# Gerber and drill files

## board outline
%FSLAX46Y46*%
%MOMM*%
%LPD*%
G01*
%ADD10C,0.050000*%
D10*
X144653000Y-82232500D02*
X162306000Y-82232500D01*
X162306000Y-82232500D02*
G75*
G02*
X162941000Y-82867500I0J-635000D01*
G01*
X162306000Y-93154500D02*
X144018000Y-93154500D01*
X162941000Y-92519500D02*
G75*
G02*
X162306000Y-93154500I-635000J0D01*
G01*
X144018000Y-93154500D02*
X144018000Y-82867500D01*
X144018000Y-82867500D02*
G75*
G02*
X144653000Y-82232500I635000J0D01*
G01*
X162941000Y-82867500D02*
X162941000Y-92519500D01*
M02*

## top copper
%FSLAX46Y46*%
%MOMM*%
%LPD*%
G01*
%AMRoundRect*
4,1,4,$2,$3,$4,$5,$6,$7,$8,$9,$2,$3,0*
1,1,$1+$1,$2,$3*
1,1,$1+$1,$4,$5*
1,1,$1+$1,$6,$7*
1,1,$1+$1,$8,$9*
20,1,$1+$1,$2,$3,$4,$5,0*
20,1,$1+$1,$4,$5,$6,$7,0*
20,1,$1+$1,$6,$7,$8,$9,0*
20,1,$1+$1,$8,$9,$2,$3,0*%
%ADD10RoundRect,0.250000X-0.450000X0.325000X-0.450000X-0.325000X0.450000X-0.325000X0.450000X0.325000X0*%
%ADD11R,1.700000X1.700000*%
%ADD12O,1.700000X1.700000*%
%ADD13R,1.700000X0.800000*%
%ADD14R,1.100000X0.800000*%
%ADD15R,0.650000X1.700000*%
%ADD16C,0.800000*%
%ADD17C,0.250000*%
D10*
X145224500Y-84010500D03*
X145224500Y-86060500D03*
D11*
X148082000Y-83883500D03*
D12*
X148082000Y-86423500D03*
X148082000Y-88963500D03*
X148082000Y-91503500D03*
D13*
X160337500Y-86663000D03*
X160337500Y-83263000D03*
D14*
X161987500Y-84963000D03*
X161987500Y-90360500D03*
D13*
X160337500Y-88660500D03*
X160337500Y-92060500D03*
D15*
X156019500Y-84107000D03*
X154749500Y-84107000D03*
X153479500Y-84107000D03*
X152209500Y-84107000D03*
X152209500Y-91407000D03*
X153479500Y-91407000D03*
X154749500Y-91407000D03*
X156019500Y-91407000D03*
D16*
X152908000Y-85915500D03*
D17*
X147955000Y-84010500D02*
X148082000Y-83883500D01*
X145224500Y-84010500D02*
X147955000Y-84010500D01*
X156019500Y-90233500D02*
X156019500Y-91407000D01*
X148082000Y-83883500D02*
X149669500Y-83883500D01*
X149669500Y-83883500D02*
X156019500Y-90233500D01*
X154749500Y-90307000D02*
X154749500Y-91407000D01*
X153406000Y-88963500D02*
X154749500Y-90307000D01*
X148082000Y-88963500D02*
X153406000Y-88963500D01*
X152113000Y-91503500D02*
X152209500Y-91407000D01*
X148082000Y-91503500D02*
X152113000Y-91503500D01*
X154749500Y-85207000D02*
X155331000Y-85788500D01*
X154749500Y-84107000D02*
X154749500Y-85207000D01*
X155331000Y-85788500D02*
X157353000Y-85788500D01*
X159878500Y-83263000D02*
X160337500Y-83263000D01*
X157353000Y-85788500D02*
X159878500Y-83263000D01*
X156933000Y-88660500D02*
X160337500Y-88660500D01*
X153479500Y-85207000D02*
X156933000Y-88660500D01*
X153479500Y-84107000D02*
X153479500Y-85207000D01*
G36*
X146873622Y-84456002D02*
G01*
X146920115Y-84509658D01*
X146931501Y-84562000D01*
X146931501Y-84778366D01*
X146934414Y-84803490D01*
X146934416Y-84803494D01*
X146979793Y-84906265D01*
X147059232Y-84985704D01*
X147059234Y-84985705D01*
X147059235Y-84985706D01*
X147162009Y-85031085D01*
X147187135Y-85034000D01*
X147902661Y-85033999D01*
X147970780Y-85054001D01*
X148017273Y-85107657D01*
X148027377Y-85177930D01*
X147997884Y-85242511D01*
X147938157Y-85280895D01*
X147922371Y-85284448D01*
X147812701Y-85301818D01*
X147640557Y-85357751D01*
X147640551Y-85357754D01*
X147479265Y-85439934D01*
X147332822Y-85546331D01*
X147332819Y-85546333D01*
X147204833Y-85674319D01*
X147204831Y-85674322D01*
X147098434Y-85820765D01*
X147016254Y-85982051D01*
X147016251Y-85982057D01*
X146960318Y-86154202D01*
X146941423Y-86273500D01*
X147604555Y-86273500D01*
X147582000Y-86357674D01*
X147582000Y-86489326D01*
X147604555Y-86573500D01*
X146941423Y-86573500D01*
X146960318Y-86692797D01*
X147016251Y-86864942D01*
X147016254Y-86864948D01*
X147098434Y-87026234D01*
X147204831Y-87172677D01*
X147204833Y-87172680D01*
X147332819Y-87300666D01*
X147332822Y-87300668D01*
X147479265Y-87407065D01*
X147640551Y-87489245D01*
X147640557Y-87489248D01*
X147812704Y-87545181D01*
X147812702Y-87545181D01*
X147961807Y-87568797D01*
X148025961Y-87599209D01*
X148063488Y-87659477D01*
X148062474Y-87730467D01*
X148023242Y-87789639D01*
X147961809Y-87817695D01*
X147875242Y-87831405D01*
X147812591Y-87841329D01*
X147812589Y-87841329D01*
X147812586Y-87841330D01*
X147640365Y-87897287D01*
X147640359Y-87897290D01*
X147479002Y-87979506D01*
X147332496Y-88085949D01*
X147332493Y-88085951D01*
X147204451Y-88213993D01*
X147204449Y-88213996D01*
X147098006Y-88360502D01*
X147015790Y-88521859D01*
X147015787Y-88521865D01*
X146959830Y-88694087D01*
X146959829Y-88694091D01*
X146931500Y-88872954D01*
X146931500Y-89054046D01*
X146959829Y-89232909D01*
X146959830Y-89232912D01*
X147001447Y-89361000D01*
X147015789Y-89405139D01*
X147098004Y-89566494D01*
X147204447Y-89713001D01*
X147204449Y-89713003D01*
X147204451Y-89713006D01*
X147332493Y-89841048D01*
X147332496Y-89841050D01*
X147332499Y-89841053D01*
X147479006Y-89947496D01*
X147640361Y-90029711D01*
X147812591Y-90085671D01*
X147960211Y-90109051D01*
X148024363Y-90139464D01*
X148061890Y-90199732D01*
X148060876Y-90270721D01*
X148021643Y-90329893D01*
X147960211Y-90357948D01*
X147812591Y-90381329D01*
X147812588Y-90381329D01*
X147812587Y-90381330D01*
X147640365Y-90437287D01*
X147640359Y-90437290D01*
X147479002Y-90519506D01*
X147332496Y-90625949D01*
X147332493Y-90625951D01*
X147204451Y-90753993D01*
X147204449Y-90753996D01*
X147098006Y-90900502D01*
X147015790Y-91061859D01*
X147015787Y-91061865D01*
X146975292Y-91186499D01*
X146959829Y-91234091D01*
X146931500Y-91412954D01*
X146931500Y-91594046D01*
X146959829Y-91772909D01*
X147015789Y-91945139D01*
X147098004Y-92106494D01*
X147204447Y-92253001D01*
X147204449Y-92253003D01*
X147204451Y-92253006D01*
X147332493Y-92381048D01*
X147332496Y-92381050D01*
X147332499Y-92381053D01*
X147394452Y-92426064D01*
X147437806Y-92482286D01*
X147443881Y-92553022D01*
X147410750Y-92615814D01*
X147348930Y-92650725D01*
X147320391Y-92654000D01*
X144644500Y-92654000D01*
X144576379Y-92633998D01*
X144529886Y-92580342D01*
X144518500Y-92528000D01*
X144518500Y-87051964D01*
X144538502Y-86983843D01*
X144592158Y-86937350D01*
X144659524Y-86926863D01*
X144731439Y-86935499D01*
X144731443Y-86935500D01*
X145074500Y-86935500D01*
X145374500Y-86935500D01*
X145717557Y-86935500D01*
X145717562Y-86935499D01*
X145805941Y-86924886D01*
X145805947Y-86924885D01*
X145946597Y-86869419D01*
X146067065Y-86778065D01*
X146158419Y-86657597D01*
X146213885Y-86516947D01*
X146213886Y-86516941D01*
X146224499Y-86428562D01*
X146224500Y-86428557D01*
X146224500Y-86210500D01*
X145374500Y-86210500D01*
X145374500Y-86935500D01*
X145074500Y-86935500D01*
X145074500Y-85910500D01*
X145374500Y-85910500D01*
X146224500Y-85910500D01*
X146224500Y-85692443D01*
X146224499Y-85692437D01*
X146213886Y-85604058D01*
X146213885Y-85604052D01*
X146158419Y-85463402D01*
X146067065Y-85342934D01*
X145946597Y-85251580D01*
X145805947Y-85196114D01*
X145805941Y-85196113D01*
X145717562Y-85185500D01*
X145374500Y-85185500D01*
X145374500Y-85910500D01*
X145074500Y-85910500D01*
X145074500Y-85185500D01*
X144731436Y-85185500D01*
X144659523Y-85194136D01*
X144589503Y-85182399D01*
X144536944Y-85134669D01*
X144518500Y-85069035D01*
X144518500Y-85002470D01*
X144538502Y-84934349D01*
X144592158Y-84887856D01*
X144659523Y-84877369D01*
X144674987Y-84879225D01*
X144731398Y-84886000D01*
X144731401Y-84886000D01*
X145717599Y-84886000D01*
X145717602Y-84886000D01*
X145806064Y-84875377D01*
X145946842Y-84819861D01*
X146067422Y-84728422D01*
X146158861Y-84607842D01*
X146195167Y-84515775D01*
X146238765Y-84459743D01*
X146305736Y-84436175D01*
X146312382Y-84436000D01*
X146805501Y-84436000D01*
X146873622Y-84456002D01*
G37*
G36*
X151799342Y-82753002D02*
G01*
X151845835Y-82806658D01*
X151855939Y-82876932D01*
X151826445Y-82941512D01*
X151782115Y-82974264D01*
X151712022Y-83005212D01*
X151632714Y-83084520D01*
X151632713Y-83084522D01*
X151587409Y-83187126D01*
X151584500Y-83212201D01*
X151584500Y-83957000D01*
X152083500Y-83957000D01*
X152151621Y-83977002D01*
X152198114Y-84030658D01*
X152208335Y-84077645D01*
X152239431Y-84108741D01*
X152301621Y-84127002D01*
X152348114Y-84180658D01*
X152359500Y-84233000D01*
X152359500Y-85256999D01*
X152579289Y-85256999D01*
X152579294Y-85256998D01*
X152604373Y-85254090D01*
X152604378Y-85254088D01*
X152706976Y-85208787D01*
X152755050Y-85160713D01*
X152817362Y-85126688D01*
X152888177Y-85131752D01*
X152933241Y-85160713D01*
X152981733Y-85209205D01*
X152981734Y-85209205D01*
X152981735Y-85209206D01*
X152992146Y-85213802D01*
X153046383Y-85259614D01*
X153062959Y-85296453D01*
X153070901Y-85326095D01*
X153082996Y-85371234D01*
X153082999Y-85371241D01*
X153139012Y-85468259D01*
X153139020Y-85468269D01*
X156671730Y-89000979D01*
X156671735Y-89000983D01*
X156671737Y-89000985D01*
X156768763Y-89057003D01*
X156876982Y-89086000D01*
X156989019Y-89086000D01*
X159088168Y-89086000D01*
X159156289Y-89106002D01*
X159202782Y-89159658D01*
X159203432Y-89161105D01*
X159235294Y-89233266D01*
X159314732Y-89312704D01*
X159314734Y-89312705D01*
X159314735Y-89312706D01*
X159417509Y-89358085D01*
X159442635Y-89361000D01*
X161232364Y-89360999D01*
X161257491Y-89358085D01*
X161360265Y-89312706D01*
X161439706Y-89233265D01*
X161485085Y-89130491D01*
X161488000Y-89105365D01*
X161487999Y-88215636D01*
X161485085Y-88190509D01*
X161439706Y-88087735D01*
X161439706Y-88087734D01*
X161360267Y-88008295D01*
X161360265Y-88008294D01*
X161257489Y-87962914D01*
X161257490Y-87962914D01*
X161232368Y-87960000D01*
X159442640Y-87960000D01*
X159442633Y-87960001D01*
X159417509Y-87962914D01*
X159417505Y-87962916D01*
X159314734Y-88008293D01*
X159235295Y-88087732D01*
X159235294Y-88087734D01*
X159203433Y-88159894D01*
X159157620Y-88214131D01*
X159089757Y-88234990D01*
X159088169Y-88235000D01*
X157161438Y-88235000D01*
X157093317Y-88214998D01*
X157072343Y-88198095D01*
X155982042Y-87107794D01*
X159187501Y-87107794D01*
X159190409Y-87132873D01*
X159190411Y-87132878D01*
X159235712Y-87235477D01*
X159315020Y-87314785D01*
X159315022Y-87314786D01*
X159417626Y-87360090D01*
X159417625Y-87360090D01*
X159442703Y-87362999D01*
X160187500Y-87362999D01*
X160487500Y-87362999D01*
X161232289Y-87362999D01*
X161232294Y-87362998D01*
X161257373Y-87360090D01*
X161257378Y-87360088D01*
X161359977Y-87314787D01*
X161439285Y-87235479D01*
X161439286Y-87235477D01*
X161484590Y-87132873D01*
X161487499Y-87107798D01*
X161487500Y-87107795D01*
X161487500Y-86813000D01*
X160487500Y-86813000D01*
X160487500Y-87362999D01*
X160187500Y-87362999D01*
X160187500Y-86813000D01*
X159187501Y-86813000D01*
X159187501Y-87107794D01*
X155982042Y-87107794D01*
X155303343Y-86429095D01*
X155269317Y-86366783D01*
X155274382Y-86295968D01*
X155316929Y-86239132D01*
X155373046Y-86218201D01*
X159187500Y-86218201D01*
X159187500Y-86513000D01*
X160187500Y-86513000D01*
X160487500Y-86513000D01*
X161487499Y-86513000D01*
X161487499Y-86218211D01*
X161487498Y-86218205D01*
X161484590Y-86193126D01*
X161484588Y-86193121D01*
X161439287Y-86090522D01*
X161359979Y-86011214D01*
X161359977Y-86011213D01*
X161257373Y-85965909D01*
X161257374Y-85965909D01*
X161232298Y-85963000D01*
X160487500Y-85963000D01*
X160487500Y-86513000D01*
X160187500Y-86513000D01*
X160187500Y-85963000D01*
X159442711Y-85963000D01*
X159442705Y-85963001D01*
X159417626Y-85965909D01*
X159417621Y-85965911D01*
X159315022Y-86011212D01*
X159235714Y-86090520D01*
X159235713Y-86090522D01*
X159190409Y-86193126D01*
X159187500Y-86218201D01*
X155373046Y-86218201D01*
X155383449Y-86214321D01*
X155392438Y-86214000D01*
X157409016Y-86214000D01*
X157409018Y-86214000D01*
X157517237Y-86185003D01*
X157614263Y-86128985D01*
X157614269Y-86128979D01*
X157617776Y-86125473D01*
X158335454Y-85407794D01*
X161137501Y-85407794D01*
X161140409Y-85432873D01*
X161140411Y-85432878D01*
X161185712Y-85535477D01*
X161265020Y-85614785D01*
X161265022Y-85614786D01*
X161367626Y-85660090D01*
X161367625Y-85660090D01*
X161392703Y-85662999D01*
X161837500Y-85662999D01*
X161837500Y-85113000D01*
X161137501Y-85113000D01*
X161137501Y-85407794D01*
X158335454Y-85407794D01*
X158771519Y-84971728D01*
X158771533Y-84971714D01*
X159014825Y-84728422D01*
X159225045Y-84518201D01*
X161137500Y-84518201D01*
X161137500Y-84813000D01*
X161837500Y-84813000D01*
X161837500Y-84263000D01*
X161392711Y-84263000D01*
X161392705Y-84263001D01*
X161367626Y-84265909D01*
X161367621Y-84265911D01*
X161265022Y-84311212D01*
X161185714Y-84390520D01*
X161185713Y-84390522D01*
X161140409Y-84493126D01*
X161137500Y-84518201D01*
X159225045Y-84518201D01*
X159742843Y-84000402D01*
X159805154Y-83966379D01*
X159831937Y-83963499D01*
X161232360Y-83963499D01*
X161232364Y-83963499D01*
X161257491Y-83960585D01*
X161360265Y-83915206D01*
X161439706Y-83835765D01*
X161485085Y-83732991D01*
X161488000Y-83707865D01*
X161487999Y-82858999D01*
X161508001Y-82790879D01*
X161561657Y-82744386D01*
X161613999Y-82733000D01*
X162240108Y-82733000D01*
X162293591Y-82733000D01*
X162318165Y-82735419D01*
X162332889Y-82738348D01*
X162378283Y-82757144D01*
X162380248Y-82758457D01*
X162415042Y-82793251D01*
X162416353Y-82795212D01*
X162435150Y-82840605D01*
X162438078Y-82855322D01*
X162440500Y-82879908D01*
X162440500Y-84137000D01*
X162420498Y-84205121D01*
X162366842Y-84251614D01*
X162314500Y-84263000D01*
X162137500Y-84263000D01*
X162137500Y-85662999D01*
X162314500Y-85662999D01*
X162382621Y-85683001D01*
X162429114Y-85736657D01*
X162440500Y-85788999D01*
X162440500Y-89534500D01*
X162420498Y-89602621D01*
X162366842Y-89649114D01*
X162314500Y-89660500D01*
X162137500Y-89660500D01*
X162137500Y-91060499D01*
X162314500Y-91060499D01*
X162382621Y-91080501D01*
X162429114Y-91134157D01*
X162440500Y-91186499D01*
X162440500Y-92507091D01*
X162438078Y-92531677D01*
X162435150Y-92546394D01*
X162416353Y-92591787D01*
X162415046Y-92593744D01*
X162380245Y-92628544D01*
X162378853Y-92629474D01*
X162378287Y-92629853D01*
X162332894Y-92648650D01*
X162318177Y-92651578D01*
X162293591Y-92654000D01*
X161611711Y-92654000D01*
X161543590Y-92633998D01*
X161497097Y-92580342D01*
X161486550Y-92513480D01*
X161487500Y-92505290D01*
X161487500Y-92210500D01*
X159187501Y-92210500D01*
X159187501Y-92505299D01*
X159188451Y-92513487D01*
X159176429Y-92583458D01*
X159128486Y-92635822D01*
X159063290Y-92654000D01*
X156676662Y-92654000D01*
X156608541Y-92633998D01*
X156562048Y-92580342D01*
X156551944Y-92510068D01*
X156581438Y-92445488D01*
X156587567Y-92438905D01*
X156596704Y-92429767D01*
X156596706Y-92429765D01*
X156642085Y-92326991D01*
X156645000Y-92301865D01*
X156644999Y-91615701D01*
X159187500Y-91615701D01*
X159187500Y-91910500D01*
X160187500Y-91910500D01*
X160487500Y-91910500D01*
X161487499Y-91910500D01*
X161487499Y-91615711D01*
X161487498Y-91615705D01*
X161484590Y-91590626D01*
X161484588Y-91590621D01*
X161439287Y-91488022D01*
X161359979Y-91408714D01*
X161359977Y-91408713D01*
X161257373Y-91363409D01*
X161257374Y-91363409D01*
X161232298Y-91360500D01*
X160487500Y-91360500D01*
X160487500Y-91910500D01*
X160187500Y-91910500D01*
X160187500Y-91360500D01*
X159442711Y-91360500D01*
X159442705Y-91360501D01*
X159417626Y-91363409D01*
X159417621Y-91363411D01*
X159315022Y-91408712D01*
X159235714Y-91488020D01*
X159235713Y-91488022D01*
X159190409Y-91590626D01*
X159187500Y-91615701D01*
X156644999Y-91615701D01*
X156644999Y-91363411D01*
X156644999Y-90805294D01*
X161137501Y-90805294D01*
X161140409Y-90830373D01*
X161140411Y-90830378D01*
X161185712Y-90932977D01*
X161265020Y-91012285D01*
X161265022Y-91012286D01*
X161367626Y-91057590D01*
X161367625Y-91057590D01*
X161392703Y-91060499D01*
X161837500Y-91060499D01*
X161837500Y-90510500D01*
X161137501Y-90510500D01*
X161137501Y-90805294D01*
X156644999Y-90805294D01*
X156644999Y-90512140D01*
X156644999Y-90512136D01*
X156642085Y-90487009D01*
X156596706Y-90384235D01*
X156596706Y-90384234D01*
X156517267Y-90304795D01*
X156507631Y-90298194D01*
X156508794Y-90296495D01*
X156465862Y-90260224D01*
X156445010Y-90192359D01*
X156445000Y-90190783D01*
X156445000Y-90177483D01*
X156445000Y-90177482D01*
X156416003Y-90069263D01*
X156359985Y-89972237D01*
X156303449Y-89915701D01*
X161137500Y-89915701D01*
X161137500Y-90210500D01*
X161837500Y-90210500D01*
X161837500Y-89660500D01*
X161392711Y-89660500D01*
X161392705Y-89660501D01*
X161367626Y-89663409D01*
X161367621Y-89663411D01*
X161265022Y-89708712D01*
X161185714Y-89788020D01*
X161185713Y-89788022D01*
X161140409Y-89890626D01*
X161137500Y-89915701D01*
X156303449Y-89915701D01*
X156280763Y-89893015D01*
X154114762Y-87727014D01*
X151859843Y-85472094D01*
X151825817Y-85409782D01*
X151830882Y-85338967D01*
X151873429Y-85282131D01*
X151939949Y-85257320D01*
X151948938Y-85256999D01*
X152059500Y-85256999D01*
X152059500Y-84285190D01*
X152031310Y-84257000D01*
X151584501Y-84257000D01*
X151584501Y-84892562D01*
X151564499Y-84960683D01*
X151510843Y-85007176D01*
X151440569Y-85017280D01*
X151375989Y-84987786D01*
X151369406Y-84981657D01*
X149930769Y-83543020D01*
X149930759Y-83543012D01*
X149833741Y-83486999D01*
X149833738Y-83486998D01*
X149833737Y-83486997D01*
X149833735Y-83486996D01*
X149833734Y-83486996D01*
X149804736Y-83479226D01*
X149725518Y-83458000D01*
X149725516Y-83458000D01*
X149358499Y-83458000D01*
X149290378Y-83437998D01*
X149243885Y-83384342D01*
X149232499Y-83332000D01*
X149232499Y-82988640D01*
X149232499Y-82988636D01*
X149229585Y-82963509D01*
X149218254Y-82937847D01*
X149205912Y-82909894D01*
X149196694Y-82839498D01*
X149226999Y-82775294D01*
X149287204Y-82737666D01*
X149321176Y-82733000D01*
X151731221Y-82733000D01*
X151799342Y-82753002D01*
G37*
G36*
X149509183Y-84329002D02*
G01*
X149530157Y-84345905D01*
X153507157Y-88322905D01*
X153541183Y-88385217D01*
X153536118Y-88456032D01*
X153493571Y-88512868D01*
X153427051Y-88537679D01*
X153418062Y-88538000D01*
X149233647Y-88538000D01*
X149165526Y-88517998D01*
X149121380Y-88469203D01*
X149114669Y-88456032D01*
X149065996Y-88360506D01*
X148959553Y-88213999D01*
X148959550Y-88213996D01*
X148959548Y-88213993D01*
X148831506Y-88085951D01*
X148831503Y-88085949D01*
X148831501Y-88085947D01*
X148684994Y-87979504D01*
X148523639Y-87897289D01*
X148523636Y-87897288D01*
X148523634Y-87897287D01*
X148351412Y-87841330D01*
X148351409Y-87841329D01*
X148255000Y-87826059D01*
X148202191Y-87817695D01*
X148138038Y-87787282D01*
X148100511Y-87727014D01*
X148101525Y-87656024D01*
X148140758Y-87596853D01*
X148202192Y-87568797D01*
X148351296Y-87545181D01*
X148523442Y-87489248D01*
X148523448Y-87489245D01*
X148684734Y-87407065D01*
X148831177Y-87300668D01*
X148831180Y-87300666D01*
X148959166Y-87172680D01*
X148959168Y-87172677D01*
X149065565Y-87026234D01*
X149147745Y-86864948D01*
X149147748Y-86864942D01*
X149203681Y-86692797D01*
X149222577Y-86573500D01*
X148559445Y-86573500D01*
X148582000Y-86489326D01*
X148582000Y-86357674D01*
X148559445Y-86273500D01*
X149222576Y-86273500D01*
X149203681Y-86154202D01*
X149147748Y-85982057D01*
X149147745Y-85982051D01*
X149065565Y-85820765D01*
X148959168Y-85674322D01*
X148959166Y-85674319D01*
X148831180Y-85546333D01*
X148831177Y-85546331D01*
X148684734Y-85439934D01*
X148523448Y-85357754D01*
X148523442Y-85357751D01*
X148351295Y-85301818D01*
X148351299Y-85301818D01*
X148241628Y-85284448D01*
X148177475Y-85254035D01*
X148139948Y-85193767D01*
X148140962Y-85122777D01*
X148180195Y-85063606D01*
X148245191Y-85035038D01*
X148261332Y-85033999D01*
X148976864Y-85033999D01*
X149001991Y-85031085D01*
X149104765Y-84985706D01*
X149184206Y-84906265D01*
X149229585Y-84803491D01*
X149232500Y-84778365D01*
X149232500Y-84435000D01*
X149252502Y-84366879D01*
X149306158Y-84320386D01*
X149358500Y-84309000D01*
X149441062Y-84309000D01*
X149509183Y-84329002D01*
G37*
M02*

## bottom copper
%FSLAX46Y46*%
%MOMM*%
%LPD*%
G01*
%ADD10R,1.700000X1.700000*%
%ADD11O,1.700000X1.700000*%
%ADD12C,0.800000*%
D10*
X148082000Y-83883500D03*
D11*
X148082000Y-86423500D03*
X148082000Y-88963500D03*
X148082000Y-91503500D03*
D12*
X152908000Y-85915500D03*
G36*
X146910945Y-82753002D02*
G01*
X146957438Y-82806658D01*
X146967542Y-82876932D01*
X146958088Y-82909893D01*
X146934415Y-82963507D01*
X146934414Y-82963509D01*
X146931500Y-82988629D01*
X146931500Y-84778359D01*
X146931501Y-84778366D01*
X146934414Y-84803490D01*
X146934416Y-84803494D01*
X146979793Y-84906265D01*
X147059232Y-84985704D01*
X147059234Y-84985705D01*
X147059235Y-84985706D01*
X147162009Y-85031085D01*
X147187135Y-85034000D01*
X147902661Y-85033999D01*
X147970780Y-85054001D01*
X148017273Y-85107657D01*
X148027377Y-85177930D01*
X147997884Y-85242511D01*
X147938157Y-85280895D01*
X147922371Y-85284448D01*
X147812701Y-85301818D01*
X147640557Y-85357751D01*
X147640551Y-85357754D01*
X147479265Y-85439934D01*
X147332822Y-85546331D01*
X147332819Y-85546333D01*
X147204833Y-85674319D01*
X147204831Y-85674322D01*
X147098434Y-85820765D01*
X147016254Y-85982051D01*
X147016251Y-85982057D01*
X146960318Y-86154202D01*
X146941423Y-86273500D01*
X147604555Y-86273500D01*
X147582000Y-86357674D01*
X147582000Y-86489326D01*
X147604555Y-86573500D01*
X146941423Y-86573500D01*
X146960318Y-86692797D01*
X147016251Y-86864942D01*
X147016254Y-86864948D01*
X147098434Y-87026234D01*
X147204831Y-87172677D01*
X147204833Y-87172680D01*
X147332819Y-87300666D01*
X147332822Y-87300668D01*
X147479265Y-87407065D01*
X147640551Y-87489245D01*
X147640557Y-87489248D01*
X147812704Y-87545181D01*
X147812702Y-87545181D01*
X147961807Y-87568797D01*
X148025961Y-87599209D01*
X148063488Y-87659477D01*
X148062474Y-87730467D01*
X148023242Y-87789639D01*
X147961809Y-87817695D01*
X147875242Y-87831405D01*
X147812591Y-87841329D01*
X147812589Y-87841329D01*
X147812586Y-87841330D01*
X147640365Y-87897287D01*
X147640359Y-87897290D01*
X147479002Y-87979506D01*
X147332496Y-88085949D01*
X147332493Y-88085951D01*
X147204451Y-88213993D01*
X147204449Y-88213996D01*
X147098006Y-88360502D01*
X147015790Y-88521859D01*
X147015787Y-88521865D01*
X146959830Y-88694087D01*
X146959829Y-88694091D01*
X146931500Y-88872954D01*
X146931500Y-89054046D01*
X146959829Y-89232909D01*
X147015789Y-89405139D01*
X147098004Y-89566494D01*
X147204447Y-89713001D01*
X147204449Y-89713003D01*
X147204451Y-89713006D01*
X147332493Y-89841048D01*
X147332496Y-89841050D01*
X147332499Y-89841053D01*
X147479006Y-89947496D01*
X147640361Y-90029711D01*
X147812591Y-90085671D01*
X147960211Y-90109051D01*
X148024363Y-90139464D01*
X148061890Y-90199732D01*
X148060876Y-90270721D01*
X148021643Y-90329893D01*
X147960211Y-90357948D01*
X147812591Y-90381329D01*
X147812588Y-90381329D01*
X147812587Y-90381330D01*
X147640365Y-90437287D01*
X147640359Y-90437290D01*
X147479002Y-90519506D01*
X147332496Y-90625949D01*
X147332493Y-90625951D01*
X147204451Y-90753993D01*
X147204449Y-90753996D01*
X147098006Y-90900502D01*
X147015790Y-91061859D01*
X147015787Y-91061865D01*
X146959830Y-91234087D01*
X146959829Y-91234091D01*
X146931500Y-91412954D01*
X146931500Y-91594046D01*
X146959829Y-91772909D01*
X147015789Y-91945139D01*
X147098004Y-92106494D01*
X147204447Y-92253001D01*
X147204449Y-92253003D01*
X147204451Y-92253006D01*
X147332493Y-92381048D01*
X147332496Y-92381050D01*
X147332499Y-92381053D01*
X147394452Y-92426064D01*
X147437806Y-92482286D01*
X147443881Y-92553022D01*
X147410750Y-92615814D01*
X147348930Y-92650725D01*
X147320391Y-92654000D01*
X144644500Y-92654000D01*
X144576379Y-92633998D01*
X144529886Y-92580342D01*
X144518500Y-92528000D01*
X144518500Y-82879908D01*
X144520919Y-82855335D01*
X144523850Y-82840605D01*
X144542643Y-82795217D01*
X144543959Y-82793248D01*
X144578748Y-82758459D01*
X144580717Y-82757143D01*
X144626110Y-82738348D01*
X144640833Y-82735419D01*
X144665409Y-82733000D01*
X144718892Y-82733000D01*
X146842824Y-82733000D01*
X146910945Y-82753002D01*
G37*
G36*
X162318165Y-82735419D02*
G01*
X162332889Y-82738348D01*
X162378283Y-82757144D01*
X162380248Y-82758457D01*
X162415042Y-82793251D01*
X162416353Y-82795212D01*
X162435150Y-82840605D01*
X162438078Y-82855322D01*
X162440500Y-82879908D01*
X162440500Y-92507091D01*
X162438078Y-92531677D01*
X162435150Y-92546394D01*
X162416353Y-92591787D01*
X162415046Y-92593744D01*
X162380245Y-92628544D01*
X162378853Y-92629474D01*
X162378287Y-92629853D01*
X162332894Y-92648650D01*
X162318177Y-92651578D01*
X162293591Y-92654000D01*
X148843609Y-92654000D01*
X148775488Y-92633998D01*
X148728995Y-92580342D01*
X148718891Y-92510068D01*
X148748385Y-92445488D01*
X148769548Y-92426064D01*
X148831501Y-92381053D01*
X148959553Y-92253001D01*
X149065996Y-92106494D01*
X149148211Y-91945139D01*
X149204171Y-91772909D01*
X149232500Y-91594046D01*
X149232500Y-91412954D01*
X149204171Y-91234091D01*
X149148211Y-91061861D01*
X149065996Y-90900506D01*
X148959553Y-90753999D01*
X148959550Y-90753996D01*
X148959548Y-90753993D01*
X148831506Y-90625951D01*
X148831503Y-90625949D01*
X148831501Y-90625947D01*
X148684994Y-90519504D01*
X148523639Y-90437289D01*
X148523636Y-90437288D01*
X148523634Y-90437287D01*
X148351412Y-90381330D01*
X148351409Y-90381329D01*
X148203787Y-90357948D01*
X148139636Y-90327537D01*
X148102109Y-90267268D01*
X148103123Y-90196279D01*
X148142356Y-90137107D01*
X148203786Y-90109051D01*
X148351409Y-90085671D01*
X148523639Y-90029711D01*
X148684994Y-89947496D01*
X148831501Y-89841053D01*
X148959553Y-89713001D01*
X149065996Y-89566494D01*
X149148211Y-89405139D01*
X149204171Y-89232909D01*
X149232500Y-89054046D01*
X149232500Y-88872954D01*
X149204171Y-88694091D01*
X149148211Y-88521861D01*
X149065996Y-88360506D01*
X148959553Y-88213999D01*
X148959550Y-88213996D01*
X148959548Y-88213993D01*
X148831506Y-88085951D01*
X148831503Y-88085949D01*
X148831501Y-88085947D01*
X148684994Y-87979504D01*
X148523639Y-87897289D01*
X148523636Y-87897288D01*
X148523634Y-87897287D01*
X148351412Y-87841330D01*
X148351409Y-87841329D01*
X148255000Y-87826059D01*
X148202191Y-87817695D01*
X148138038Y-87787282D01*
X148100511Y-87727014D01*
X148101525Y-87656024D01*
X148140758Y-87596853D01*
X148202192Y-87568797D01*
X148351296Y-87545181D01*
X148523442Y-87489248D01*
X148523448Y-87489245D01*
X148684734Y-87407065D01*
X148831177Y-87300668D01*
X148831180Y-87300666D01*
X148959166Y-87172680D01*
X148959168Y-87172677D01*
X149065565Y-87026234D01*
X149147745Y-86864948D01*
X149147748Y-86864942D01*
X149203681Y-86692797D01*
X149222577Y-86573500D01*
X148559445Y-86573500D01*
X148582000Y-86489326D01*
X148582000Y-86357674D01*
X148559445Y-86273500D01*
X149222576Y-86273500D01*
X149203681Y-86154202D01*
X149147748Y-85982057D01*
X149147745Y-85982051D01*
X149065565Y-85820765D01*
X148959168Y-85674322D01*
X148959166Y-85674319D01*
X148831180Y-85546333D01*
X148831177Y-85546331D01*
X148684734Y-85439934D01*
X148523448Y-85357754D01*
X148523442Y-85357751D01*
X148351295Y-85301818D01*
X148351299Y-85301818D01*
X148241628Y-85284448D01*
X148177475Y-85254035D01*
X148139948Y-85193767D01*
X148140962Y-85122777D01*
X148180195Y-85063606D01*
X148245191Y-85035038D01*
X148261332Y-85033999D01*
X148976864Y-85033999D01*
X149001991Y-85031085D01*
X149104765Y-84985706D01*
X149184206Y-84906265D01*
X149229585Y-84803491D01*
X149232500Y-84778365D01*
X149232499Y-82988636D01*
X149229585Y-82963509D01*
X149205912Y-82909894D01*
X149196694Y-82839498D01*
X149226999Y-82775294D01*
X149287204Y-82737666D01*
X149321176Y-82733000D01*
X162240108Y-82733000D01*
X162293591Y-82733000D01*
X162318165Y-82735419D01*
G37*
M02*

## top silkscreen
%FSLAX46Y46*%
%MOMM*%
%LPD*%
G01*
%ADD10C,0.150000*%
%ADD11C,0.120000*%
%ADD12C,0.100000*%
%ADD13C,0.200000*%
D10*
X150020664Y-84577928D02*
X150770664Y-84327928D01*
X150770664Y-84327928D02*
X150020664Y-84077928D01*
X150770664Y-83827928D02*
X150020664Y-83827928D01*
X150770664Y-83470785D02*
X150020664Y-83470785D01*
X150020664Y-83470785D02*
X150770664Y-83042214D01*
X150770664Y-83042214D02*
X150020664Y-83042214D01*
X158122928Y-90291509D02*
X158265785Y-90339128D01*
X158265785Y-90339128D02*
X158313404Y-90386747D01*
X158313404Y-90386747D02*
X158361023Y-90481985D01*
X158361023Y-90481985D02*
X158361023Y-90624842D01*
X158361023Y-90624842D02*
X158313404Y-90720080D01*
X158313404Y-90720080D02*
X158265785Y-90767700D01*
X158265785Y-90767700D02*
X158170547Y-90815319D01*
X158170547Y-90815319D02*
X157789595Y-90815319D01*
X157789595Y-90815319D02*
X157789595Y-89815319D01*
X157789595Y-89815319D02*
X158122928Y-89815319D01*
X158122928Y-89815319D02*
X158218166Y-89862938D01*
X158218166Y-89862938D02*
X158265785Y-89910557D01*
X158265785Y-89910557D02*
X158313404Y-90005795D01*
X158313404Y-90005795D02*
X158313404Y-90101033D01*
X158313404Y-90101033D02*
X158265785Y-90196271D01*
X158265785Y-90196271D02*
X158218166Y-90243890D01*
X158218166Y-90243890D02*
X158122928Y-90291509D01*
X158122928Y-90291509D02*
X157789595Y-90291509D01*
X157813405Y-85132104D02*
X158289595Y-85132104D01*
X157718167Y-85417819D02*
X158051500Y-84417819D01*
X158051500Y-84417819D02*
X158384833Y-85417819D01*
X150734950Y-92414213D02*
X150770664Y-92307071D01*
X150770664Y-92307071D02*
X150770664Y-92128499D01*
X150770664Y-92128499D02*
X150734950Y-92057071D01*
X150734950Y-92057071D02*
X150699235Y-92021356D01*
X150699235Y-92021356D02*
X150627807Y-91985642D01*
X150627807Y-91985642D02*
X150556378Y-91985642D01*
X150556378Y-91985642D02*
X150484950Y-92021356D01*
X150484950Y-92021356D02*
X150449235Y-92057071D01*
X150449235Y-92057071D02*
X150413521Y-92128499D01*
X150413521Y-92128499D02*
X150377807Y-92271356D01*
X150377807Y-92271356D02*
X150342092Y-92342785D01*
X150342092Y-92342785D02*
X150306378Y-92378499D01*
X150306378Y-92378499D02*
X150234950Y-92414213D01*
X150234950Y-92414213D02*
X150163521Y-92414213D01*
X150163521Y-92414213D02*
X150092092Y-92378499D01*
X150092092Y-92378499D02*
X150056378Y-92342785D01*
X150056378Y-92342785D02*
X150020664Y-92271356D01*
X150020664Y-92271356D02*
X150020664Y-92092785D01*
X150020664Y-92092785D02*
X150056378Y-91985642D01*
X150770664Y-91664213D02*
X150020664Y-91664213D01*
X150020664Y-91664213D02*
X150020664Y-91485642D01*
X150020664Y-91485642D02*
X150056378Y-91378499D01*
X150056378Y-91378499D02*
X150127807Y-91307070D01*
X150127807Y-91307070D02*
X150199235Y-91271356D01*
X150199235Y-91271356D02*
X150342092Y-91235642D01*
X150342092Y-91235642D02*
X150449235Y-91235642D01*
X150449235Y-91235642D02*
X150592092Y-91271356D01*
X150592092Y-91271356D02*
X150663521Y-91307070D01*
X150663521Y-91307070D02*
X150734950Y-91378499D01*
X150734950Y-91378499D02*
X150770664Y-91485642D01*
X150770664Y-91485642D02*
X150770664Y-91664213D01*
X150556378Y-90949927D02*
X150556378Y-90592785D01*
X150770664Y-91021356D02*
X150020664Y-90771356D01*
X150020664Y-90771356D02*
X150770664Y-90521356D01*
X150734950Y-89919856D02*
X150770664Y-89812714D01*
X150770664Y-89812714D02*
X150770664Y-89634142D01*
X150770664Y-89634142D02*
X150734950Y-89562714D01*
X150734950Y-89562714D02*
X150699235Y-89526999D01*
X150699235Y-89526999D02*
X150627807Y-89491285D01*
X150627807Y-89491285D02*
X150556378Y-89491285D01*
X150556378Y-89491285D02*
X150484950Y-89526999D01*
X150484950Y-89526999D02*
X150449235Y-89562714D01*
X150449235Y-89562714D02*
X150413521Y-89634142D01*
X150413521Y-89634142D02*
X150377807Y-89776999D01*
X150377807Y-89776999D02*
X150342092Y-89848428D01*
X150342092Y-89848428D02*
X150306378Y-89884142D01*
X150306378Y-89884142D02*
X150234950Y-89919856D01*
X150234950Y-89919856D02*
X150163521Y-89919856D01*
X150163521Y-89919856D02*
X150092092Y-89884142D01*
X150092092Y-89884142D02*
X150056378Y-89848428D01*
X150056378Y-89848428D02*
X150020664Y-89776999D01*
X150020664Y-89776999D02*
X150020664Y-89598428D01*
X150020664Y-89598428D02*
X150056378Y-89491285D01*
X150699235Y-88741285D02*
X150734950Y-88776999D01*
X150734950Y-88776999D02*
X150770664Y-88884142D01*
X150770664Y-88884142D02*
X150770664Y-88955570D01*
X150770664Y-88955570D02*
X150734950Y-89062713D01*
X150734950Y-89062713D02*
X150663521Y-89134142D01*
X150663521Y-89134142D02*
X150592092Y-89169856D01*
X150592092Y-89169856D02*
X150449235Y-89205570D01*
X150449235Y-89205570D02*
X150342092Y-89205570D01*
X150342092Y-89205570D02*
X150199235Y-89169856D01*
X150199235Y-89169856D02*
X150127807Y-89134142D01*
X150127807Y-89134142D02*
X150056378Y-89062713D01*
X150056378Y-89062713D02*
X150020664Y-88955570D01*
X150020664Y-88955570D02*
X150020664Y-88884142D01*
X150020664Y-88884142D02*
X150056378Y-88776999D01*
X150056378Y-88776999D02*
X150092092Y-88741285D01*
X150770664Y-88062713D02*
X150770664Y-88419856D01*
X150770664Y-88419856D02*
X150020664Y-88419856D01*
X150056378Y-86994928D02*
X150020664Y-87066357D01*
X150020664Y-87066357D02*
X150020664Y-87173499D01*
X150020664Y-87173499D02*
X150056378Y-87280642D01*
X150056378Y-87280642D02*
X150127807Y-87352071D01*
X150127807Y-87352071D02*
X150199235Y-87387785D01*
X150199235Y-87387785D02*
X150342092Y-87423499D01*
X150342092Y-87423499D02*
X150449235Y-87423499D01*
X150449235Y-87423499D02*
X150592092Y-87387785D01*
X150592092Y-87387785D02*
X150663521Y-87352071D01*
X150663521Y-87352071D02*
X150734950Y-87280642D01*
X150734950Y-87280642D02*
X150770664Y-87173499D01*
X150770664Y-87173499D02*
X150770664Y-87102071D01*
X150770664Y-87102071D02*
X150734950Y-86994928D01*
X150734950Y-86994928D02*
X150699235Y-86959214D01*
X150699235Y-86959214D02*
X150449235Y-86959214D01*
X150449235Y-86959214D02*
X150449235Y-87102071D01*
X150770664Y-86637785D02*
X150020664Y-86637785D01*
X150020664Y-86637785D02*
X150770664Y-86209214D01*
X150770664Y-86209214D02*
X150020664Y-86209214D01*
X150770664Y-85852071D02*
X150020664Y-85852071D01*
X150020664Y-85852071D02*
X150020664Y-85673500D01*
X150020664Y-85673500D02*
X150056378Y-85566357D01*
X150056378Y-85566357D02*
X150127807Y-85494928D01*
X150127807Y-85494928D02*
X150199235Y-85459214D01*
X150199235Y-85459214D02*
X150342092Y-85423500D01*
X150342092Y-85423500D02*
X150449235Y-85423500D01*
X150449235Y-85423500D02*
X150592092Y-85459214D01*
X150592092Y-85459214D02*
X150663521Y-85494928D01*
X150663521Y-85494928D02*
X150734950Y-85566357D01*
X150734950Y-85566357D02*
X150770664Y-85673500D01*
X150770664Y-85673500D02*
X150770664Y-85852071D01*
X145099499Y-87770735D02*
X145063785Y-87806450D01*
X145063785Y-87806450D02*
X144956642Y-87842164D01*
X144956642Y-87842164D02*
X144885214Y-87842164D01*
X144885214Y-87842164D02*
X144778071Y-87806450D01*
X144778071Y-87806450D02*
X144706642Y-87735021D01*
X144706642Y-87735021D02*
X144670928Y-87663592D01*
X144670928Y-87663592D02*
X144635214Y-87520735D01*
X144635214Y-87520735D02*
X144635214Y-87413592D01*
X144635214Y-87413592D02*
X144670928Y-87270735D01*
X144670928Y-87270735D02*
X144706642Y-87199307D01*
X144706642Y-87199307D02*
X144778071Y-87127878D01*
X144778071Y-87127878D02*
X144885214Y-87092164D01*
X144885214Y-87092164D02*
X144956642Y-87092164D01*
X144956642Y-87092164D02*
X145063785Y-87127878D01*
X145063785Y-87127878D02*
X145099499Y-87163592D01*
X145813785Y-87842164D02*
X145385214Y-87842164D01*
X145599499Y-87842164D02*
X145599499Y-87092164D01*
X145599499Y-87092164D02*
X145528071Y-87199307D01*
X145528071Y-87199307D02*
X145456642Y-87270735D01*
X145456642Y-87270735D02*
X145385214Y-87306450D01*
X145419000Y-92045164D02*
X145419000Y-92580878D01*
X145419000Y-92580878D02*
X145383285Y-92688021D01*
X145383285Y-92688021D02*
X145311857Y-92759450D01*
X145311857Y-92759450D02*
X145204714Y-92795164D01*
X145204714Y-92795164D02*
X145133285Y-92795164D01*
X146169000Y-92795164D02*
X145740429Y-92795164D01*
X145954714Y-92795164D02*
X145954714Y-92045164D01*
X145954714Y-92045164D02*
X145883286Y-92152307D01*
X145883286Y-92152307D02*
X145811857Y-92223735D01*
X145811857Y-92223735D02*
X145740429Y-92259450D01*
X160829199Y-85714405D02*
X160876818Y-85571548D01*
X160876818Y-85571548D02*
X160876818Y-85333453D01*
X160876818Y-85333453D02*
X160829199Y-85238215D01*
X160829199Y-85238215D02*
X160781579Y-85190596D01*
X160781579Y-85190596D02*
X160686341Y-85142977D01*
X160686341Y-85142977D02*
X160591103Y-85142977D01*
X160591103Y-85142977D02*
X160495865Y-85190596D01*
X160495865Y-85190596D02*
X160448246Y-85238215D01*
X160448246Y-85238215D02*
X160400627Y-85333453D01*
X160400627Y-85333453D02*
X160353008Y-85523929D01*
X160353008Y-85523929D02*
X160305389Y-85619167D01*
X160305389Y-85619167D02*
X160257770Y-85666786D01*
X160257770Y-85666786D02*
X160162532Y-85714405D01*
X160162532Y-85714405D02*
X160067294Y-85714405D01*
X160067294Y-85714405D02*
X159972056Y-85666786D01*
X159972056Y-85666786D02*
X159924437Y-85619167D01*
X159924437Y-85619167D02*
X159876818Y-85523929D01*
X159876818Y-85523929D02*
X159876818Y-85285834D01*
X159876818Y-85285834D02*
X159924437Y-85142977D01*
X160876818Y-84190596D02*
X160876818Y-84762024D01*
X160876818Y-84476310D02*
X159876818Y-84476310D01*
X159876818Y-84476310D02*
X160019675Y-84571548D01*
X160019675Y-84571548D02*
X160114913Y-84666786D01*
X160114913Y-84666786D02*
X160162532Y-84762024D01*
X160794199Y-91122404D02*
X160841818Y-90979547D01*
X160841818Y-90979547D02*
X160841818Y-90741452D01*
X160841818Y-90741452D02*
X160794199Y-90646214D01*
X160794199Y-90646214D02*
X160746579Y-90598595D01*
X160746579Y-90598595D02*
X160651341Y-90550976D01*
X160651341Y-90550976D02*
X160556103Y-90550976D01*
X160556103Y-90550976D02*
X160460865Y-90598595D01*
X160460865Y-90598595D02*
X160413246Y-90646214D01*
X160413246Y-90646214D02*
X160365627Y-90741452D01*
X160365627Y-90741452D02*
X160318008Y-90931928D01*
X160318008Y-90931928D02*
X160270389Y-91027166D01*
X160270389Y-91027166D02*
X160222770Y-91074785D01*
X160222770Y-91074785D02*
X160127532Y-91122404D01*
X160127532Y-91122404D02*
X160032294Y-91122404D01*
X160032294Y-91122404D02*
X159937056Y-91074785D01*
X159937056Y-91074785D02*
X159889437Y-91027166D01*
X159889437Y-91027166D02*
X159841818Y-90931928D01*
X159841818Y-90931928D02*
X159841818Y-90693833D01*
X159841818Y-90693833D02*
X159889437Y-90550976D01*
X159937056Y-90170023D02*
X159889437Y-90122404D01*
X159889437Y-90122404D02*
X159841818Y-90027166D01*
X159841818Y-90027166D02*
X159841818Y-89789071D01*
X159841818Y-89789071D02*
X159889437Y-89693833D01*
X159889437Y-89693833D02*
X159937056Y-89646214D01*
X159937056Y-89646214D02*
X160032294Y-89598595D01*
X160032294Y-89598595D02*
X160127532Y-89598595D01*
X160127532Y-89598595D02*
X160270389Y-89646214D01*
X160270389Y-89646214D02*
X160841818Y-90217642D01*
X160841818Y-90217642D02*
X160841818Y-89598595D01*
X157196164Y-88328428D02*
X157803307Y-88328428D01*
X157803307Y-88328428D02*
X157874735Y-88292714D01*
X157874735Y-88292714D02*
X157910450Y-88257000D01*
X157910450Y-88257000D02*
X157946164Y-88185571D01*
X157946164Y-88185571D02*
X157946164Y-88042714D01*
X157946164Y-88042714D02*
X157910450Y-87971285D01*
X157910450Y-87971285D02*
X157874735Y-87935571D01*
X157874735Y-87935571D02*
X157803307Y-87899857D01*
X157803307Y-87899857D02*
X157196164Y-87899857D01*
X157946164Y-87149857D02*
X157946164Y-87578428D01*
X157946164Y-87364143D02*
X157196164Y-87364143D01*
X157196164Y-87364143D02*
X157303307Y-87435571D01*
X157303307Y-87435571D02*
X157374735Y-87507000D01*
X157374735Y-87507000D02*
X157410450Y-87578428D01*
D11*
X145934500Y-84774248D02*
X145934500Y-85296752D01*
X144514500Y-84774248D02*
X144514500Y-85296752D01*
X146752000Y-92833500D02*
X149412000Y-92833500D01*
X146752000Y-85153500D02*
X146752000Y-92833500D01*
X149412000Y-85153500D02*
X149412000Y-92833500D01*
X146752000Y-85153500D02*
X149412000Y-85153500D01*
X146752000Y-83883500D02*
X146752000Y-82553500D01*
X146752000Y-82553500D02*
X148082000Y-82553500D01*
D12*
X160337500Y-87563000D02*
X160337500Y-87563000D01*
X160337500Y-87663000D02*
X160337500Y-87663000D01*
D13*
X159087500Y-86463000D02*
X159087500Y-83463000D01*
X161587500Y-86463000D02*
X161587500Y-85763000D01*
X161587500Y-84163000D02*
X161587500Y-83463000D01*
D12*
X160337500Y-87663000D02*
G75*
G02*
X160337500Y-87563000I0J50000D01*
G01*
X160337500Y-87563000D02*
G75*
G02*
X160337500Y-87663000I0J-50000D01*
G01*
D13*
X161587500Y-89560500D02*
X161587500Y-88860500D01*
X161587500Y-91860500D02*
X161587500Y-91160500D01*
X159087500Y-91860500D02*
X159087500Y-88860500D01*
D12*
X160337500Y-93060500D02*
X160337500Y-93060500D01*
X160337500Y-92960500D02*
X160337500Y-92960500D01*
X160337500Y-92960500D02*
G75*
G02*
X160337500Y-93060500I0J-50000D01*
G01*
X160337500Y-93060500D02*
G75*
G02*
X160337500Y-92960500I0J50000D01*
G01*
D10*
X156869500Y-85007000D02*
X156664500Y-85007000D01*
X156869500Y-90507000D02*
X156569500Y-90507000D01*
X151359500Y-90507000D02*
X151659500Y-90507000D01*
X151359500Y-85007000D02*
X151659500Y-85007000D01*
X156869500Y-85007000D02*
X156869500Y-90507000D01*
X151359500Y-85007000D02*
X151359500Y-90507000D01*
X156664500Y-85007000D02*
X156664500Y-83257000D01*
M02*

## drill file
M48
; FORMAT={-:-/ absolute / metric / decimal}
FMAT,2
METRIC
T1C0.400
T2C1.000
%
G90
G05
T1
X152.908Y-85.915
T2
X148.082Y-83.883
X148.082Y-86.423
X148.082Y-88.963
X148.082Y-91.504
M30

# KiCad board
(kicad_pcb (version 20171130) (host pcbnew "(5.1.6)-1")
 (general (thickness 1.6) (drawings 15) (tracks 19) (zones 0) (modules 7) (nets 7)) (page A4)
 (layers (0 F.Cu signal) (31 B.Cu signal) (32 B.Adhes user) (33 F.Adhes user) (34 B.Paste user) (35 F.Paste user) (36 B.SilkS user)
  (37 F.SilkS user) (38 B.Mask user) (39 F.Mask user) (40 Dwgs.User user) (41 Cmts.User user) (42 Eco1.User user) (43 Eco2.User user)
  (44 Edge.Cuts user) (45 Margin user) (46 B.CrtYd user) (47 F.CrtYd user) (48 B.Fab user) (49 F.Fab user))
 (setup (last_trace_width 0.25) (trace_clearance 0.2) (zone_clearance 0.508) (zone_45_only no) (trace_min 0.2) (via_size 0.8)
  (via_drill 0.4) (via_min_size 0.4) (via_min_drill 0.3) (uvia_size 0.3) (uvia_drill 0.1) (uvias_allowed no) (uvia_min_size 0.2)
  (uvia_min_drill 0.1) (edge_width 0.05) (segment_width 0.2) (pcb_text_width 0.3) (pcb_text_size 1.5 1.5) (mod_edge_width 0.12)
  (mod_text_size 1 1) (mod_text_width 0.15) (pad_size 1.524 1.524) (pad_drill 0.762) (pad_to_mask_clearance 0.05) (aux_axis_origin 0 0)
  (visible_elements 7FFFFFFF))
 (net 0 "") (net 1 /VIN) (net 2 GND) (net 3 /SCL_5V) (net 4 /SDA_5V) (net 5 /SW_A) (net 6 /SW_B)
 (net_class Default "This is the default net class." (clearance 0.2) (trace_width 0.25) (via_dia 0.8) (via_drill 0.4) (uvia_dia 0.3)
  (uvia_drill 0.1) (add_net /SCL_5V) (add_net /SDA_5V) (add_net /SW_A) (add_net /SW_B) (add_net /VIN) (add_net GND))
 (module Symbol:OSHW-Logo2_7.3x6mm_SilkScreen (layer B.Cu) (at 159.512 88.519 180)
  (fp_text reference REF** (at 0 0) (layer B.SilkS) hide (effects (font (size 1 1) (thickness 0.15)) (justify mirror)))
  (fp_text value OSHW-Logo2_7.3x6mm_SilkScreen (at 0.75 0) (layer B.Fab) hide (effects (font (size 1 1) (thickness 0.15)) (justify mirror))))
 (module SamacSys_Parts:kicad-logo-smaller (layer B.Cu) (at 153.0985 88.265 180)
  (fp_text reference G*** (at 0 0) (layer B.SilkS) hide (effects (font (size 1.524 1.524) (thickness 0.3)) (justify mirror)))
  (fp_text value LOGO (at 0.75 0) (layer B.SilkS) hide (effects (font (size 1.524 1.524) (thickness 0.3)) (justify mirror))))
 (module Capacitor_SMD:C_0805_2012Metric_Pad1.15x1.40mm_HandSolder (layer F.Cu) (at 145.2245 85.0355 270)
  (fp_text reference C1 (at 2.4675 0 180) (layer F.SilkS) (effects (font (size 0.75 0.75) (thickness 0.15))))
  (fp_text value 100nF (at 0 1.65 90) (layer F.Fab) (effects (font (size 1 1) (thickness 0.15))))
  (fp_line (start -0.261252 -0.71) (end 0.261252 -0.71) (layer F.SilkS) (width 0.12))
  (fp_line (start -0.261252 0.71) (end 0.261252 0.71) (layer F.SilkS) (width 0.12))
  (pad 1 smd roundrect (at -1.025 0 270) (size 1.15 1.4) (layers F.Cu F.Paste F.Mask) (roundrect_rratio 0.217391) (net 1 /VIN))
  (pad 2 smd roundrect (at 1.025 0 270) (size 1.15 1.4) (layers F.Cu F.Paste F.Mask) (roundrect_rratio 0.217391) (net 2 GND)))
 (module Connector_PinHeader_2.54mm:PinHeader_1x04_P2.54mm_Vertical (layer F.Cu) (at 148.082 83.8835)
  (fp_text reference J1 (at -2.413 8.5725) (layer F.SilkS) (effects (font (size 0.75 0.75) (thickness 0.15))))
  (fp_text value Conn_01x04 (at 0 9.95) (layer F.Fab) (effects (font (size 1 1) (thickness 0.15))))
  (fp_line (start -1.33 8.95) (end 1.33 8.95) (layer F.SilkS) (width 0.12))
  (fp_line (start -1.33 1.27) (end -1.33 8.95) (layer F.SilkS) (width 0.12))
  (fp_line (start 1.33 1.27) (end 1.33 8.95) (layer F.SilkS) (width 0.12))
  (fp_line (start -1.33 1.27) (end 1.33 1.27) (layer F.SilkS) (width 0.12))
  (fp_line (start -1.33 0) (end -1.33 -1.33) (layer F.SilkS) (width 0.12))
  (fp_line (start -1.33 -1.33) (end 0 -1.33) (layer F.SilkS) (width 0.12))
  (pad 1 thru_hole rect (at 0 0) (size 1.7 1.7) (drill 1) (layers *.Cu *.Mask) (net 1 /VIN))
  (pad 2 thru_hole oval (at 0 2.54) (size 1.7 1.7) (drill 1) (layers *.Cu *.Mask) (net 2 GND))
  (pad 3 thru_hole oval (at 0 5.08) (size 1.7 1.7) (drill 1) (layers *.Cu *.Mask) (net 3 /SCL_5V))
  (pad 4 thru_hole oval (at 0 7.62) (size 1.7 1.7) (drill 1) (layers *.Cu *.Mask) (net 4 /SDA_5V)))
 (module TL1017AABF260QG (layer F.Cu) (at 160.3375 84.963 90)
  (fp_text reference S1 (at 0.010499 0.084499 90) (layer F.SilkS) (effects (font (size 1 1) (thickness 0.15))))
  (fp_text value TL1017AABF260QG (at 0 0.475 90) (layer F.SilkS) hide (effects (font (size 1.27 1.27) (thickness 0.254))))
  (fp_line (start -2.6 0) (end -2.6 0) (layer F.SilkS) (width 0.1))
  (fp_line (start -2.7 0) (end -2.7 0) (layer F.SilkS) (width 0.1))
  (fp_line (start -1.5 -1.25) (end 1.5 -1.25) (layer F.SilkS) (width 0.2))
  (fp_line (start -1.5 1.25) (end -0.8 1.25) (layer F.SilkS) (width 0.2))
  (fp_line (start 0.8 1.25) (end 1.5 1.25) (layer F.SilkS) (width 0.2))
  (fp_arc (start -2.65 0) (end -2.6 0) (angle -180) (layer F.SilkS) (width 0.1))
  (fp_arc (start -2.65 0) (end -2.7 0) (angle -180) (layer F.SilkS) (width 0.1))
  (pad 1 smd rect (at -1.7 0 90) (size 0.8 1.7) (layers F.Cu F.Paste F.Mask) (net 2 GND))
  (pad 2 smd rect (at 1.7 0 90) (size 0.8 1.7) (layers F.Cu F.Paste F.Mask) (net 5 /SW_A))
  (pad G1 smd rect (at 0 1.65 90) (size 0.8 1.1) (layers F.Cu F.Paste F.Mask) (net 2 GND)))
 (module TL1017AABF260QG (layer F.Cu) (at 160.3375 90.3605 90)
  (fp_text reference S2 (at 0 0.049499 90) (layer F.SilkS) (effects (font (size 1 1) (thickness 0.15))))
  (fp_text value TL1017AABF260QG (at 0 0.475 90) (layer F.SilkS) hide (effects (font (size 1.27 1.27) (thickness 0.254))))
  (fp_line (start 0.8 1.25) (end 1.5 1.25) (layer F.SilkS) (width 0.2))
  (fp_line (start -1.5 1.25) (end -0.8 1.25) (layer F.SilkS) (width 0.2))
  (fp_line (start -1.5 -1.25) (end 1.5 -1.25) (layer F.SilkS) (width 0.2))
  (fp_line (start -2.7 0) (end -2.7 0) (layer F.SilkS) (width 0.1))
  (fp_line (start -2.6 0) (end -2.6 0) (layer F.SilkS) (width 0.1))
  (fp_arc (start -2.65 0) (end -2.7 0) (angle -180) (layer F.SilkS) (width 0.1))
  (fp_arc (start -2.65 0) (end -2.6 0) (angle -180) (layer F.SilkS) (width 0.1))
  (pad G1 smd rect (at 0 1.65 90) (size 0.8 1.1) (layers F.Cu F.Paste F.Mask) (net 2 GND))
  (pad 2 smd rect (at 1.7 0 90) (size 0.8 1.7) (layers F.Cu F.Paste F.Mask) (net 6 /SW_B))
  (pad 1 smd rect (at -1.7 0 90) (size 0.8 1.7) (layers F.Cu F.Paste F.Mask) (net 2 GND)))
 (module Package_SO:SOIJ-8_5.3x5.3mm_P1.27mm (layer F.Cu) (at 154.1145 87.757 270)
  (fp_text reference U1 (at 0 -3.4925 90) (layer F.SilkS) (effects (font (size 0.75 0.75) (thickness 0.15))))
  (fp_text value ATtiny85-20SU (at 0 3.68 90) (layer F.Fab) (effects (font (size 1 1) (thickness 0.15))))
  (fp_line (start -2.75 -2.755) (end -2.75 -2.55) (layer F.SilkS) (width 0.15))
  (fp_line (start 2.75 -2.755) (end 2.75 -2.455) (layer F.SilkS) (width 0.15))
  (fp_line (start 2.75 2.755) (end 2.75 2.455) (layer F.SilkS) (width 0.15))
  (fp_line (start -2.75 2.755) (end -2.75 2.455) (layer F.SilkS) (width 0.15))
  (fp_line (start -2.75 -2.755) (end 2.75 -2.755) (layer F.SilkS) (width 0.15))
  (fp_line (start -2.75 2.755) (end 2.75 2.755) (layer F.SilkS) (width 0.15))
  (fp_line (start -2.75 -2.55) (end -4.5 -2.55) (layer F.SilkS) (width 0.15))
  (pad 1 smd rect (at -3.65 -1.905 270) (size 1.7 0.65) (layers F.Cu F.Paste F.Mask))
  (pad 2 smd rect (at -3.65 -0.635 270) (size 1.7 0.65) (layers F.Cu F.Paste F.Mask) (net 5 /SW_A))
  (pad 3 smd rect (at -3.65 0.635 270) (size 1.7 0.65) (layers F.Cu F.Paste F.Mask) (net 6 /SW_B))
  (pad 4 smd rect (at -3.65 1.905 270) (size 1.7 0.65) (layers F.Cu F.Paste F.Mask) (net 2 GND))
  (pad 5 smd rect (at 3.65 1.905 270) (size 1.7 0.65) (layers F.Cu F.Paste F.Mask) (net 4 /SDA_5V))
  (pad 6 smd rect (at 3.65 0.635 270) (size 1.7 0.65) (layers F.Cu F.Paste F.Mask))
  (pad 7 smd rect (at 3.65 -0.635 270) (size 1.7 0.65) (layers F.Cu F.Paste F.Mask) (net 3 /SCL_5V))
  (pad 8 smd rect (at 3.65 -1.905 270) (size 1.7 0.65) (layers F.Cu F.Paste F.Mask) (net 1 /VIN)))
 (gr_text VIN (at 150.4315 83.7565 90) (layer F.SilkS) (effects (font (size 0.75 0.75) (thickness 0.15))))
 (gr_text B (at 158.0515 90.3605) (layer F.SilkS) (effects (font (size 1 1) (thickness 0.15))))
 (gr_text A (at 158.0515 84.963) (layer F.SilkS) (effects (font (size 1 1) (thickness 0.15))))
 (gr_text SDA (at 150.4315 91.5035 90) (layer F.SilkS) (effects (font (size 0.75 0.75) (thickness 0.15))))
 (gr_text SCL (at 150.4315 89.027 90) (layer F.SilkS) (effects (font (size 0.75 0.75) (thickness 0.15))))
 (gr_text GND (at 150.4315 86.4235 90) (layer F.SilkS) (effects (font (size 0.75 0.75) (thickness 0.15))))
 (gr_line (start 144.653 82.2325) (end 162.306 82.2325) (layer Edge.Cuts) (width 0.05))
 (gr_arc (start 162.306 82.8675) (end 162.941 82.8675) (angle -90) (layer Edge.Cuts) (width 0.05))
 (gr_line (start 162.306 93.1545) (end 144.018 93.1545) (layer Edge.Cuts) (width 0.05))
 (gr_arc (start 162.306 92.5195) (end 162.306 93.1545) (angle -90) (layer Edge.Cuts) (width 0.05))
 (gr_line (start 144.018 93.1545) (end 144.018 82.8675) (layer Edge.Cuts) (width 0.05))
 (gr_arc (start 144.653 82.8675) (end 144.653 82.2325) (angle -90) (layer Edge.Cuts) (width 0.05))
 (gr_line (start 162.941 82.8675) (end 162.941 92.5195) (layer Edge.Cuts) (width 0.05))
 (segment (start 147.955 84.0105) (end 148.082 83.8835) (width 0.25) (layer F.Cu) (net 1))
 (segment (start 145.2245 84.0105) (end 147.955 84.0105) (width 0.25) (layer F.Cu) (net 1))
 (segment (start 156.0195 90.2335) (end 156.0195 91.407) (width 0.25) (layer F.Cu) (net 1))
 (segment (start 148.082 83.8835) (end 149.6695 83.8835) (width 0.25) (layer F.Cu) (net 1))
 (segment (start 149.6695 83.8835) (end 156.0195 90.2335) (width 0.25) (layer F.Cu) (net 1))
 (via (at 152.908 85.9155) (size 0.8) (drill 0.4) (layers F.Cu B.Cu) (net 2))
 (segment (start 154.7495 90.307) (end 154.7495 91.407) (width 0.25) (layer F.Cu) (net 3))
 (segment (start 153.406 88.9635) (end 154.7495 90.307) (width 0.25) (layer F.Cu) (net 3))
 (segment (start 148.082 88.9635) (end 153.406 88.9635) (width 0.25) (layer F.Cu) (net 3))
 (segment (start 152.113 91.5035) (end 152.2095 91.407) (width 0.25) (layer F.Cu) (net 4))
 (segment (start 148.082 91.5035) (end 152.113 91.5035) (width 0.25) (layer F.Cu) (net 4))
 (segment (start 154.7495 85.207) (end 155.331 85.7885) (width 0.25) (layer F.Cu) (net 5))
 (segment (start 154.7495 84.107) (end 154.7495 85.207) (width 0.25) (layer F.Cu) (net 5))
 (segment (start 155.331 85.7885) (end 157.353 85.7885) (width 0.25) (layer F.Cu) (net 5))
 (segment (start 159.8785 83.263) (end 160.3375 83.263) (width 0.25) (layer F.Cu) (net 5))
 (segment (start 157.353 85.7885) (end 159.8785 83.263) (width 0.25) (layer F.Cu) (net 5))
 (segment (start 156.933 88.6605) (end 160.3375 88.6605) (width 0.25) (layer F.Cu) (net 6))
 (segment (start 153.4795 85.207) (end 156.933 88.6605) (width 0.25) (layer F.Cu) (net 6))
 (segment (start 153.4795 84.107) (end 153.4795 85.207) (width 0.25) (layer F.Cu) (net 6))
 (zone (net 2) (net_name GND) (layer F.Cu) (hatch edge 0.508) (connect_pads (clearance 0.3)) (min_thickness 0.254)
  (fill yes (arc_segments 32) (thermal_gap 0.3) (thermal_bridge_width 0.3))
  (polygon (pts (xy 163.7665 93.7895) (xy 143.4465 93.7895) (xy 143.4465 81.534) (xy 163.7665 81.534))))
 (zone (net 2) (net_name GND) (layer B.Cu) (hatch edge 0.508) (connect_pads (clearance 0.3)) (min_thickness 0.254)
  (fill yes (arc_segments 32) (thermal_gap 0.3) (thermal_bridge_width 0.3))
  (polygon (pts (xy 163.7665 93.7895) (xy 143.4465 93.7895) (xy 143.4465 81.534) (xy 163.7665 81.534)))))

